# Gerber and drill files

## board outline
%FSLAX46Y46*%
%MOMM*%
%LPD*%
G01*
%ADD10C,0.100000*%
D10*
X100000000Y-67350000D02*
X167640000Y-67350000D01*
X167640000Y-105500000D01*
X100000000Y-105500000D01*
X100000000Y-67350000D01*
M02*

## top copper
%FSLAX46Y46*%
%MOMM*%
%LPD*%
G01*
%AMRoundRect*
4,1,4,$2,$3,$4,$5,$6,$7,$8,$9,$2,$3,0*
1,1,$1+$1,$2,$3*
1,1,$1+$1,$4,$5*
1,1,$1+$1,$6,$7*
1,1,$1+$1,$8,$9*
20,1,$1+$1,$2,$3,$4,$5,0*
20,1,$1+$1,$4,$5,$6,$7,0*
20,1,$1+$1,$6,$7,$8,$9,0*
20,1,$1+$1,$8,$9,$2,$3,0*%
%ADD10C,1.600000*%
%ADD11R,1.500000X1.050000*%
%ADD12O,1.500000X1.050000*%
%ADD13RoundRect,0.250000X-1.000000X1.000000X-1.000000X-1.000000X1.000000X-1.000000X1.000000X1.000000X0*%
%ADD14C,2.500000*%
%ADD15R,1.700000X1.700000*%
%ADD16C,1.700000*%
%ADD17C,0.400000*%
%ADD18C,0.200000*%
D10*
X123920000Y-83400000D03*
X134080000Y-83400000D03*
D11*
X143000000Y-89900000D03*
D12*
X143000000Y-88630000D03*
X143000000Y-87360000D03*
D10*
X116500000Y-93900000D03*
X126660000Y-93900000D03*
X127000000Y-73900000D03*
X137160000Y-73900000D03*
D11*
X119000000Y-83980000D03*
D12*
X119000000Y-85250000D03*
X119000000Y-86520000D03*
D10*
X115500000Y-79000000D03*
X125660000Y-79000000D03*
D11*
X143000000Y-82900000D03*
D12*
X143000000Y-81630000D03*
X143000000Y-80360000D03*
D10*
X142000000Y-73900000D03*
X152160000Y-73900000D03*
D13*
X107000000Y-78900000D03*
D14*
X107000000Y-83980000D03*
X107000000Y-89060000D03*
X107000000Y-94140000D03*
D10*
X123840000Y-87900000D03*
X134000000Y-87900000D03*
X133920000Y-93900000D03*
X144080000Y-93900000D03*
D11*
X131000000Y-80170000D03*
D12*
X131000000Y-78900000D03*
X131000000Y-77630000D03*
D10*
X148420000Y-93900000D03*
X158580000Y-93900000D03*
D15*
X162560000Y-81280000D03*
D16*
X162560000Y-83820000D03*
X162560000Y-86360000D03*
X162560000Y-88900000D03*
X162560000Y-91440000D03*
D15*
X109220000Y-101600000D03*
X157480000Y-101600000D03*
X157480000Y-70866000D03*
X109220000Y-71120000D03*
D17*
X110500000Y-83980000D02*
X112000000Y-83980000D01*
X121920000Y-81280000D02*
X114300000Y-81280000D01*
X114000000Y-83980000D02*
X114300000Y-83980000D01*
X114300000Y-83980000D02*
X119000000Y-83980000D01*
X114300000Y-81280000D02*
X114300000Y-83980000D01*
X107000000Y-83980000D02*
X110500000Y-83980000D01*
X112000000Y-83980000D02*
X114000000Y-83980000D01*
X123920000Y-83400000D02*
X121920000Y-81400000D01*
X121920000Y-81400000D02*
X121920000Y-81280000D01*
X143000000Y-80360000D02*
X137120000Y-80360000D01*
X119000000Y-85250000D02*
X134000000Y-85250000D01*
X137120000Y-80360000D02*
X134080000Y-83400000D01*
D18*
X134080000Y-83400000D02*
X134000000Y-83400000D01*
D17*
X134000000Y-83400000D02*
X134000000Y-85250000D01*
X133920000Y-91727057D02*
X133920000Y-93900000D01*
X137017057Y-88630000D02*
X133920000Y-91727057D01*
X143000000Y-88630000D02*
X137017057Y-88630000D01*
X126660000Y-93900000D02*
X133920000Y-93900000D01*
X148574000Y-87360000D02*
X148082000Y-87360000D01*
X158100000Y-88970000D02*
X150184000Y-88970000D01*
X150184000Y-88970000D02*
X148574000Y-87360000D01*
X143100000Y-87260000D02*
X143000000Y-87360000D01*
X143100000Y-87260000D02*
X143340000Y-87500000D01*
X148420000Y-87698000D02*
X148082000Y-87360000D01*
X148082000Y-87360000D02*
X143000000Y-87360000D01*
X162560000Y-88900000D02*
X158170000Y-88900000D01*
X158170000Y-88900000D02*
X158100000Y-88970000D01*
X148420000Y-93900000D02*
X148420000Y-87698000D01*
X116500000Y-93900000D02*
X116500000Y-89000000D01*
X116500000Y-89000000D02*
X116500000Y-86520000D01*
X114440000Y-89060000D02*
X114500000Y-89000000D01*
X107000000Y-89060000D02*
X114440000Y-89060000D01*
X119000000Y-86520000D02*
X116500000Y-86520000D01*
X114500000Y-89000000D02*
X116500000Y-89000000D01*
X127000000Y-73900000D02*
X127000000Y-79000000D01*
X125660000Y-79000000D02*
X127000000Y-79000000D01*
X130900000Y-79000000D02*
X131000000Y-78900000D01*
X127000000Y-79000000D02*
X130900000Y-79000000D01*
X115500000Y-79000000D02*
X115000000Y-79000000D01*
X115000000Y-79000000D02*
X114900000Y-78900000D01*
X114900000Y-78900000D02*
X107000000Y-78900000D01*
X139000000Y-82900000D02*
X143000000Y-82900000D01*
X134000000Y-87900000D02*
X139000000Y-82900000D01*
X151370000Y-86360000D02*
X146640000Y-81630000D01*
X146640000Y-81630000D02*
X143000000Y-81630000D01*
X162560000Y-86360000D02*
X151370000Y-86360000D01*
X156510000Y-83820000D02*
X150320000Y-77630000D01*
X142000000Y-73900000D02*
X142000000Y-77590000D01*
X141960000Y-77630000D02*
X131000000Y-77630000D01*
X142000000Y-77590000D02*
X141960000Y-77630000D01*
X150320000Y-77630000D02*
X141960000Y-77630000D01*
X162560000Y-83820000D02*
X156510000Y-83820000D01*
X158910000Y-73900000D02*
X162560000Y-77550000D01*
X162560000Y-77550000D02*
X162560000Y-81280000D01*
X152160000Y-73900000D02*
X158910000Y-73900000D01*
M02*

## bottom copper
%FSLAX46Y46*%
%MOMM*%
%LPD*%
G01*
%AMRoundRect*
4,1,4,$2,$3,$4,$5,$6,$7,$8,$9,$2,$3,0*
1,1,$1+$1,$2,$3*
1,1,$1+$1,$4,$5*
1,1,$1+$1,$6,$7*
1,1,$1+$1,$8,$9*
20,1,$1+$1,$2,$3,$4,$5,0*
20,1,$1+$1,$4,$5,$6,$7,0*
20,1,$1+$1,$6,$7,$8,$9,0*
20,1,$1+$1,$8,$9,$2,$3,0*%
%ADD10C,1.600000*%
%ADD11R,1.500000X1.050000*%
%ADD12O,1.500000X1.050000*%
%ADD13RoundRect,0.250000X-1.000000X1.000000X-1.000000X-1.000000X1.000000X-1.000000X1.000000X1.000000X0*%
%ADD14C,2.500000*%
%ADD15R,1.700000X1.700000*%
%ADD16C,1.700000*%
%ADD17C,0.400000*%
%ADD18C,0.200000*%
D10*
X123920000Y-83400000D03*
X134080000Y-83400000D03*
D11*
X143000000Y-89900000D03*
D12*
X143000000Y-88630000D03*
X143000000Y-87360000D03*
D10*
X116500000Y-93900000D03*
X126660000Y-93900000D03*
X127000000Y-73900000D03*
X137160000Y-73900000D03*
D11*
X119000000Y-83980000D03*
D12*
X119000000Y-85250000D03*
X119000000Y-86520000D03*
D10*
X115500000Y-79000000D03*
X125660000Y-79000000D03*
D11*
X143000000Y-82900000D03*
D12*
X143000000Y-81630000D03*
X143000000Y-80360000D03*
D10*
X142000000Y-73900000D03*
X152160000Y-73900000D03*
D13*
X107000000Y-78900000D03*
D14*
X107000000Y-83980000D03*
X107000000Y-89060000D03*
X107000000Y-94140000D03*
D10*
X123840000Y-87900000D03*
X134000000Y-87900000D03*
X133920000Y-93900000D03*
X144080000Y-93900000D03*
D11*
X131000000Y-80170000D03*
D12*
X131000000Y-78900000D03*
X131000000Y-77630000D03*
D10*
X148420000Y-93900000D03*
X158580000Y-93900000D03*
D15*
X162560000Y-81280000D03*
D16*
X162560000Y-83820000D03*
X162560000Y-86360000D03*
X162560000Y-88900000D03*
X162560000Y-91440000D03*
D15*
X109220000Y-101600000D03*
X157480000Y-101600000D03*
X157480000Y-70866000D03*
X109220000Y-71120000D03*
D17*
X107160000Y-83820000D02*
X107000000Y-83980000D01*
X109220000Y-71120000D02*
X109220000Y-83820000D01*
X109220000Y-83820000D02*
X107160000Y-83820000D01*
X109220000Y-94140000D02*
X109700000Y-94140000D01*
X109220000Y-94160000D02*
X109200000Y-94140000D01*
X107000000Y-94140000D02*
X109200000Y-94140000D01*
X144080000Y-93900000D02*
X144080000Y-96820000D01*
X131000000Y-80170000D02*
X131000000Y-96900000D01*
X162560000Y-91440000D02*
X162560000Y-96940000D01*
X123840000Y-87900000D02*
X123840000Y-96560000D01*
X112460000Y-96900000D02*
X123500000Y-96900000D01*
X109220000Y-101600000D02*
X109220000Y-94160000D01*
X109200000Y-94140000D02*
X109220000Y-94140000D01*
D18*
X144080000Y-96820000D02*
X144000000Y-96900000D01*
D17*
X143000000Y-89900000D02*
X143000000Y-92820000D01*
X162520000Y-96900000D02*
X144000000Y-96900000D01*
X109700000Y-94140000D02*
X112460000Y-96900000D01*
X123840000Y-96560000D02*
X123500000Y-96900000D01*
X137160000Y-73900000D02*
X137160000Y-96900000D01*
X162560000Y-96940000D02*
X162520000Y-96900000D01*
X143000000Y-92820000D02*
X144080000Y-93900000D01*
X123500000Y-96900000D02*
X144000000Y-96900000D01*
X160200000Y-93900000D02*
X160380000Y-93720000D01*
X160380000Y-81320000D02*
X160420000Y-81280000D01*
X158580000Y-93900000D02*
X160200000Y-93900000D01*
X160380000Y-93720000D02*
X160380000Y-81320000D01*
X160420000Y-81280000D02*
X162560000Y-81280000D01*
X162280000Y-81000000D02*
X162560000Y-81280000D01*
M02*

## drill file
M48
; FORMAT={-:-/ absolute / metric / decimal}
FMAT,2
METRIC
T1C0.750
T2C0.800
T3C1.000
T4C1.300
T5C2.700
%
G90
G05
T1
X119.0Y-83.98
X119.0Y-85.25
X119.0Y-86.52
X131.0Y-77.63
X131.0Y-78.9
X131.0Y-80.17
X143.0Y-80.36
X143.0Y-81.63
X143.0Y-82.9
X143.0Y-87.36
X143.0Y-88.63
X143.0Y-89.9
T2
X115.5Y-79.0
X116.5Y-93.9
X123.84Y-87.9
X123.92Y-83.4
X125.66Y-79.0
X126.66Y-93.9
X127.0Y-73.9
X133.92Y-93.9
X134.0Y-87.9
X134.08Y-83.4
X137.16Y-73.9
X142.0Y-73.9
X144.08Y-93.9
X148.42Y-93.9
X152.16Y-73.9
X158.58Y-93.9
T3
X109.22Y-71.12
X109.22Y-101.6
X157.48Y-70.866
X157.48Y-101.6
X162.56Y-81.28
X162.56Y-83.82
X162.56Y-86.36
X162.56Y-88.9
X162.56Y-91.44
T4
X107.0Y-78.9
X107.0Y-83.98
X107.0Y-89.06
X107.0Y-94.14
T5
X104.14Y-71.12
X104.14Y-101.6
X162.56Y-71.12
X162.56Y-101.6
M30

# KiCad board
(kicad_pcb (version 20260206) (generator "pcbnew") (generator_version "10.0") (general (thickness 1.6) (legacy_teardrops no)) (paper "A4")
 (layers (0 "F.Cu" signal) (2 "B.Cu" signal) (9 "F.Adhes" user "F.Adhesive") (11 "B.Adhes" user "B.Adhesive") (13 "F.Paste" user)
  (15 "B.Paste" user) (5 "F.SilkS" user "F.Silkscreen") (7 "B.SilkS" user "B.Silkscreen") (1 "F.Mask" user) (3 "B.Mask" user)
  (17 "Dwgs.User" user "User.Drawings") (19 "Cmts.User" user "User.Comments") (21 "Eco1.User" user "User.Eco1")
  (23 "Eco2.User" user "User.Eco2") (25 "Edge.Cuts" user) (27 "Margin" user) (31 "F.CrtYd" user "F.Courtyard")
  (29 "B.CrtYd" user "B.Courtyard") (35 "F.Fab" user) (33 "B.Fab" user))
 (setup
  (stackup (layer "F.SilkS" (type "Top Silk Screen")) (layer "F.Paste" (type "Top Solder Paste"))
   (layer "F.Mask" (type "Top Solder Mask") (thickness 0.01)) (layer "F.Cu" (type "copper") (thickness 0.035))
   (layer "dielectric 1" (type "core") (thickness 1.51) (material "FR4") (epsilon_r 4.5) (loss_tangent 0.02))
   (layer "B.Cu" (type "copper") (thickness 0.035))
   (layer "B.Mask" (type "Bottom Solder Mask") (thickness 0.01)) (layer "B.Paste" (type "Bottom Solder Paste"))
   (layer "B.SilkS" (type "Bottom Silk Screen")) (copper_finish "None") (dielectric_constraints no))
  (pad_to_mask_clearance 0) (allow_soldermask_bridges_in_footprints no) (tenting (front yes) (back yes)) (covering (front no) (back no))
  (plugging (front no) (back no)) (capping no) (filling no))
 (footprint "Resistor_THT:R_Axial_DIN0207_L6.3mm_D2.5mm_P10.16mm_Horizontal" (layer "F.Cu") (at 123.92 83.4)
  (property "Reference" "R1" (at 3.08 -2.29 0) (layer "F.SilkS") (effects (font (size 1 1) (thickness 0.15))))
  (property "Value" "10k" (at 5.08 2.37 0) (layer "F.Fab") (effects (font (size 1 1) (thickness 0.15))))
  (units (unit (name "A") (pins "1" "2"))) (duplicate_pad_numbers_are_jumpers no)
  (pad "1" thru_hole circle (at 0 0) (size 1.6 1.6) (drill 0.8) (layers "*.Cu" "*.Mask") (remove_unused_layers no) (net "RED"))
  (pad "2" thru_hole circle (at 10.16 0) (size 1.6 1.6) (drill 0.8) (layers "*.Cu" "*.Mask") (remove_unused_layers no) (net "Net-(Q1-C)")))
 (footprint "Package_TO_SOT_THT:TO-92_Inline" (layer "F.Cu") (at 143 89.9 90)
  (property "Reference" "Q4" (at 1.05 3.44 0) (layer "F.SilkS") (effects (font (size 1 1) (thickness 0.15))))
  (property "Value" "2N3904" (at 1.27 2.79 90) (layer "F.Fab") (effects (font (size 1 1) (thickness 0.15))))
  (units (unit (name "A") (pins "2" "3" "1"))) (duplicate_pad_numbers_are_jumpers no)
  (pad "1" thru_hole rect (at 0 0 90) (size 1.05 1.5) (drill 0.75) (layers "*.Cu" "*.Mask") (remove_unused_layers no) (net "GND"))
  (pad "2" thru_hole oval (at 1.27 0 90) (size 1.05 1.5) (drill 0.75) (layers "*.Cu" "*.Mask") (remove_unused_layers no) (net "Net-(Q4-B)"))
  (pad "3" thru_hole oval (at 2.54 0 90) (size 1.05 1.5) (drill 0.75) (layers "*.Cu" "*.Mask") (remove_unused_layers no) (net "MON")))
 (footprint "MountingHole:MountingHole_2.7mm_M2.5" (layer "F.Cu") (at 162.56 101.6)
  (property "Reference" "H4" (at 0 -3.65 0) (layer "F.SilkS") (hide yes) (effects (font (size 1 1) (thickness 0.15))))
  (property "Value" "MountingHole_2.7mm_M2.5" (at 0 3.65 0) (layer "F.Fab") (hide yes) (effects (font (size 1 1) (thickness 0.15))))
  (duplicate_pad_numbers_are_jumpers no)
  (pad "" np_thru_hole circle (at 0 0) (size 2.7 2.7) (drill 2.7) (layers "*.Cu" "*.Mask")))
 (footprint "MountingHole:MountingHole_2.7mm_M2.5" (layer "F.Cu") (at 104.14 71.12)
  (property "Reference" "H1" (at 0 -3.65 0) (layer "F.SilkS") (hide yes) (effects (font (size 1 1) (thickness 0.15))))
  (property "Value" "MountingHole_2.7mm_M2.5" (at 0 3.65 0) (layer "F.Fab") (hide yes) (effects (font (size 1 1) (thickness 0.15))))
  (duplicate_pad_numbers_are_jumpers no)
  (pad "" np_thru_hole circle (at 0 0) (size 2.7 2.7) (drill 2.7) (layers "*.Cu" "*.Mask")))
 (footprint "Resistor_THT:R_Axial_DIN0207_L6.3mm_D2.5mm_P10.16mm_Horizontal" (layer "F.Cu") (at 116.5 93.9)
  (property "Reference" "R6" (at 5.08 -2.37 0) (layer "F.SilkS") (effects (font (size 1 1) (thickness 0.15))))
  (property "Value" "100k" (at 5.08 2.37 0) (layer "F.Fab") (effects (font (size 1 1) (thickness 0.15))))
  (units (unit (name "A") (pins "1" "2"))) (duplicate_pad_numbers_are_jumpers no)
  (pad "1" thru_hole circle (at 0 0) (size 1.6 1.6) (drill 0.8) (layers "*.Cu" "*.Mask") (remove_unused_layers no) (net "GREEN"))
  (pad "2" thru_hole circle (at 10.16 0) (size 1.6 1.6) (drill 0.8) (layers "*.Cu" "*.Mask") (remove_unused_layers no) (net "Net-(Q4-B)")))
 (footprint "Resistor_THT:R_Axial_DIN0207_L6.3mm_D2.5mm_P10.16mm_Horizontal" (layer "F.Cu") (at 127 73.9)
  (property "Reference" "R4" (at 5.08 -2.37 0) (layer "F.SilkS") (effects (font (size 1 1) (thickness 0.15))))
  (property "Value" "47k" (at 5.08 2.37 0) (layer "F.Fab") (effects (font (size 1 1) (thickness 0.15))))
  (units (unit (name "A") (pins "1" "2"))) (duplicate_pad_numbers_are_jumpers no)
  (pad "1" thru_hole circle (at 0 0) (size 1.6 1.6) (drill 0.8) (layers "*.Cu" "*.Mask") (remove_unused_layers no) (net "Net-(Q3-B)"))
  (pad "2" thru_hole circle (at 10.16 0) (size 1.6 1.6) (drill 0.8) (layers "*.Cu" "*.Mask") (remove_unused_layers no) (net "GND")))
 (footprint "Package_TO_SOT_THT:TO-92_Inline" (layer "F.Cu") (at 119 83.98 -90)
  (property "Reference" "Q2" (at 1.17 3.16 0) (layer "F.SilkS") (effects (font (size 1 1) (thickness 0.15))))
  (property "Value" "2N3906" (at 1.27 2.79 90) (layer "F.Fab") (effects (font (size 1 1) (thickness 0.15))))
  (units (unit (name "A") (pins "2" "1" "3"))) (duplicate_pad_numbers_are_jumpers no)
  (pad "1" thru_hole rect (at 0 0 270) (size 1.05 1.5) (drill 0.75) (layers "*.Cu" "*.Mask") (remove_unused_layers no) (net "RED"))
  (pad "2" thru_hole oval (at 1.27 0 270) (size 1.05 1.5) (drill 0.75) (layers "*.Cu" "*.Mask") (remove_unused_layers no) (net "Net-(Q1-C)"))
  (pad "3" thru_hole oval (at 2.54 0 270) (size 1.05 1.5) (drill 0.75) (layers "*.Cu" "*.Mask") (remove_unused_layers no) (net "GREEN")))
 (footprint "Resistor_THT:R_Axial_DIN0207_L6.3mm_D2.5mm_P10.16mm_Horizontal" (layer "F.Cu") (at 115.5 79)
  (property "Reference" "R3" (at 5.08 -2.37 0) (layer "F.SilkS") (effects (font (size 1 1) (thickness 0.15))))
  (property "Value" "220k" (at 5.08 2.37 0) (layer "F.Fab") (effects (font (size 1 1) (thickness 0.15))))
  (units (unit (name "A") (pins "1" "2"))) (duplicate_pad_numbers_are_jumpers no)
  (pad "1" thru_hole circle (at 0 0) (size 1.6 1.6) (drill 0.8) (layers "*.Cu" "*.Mask") (remove_unused_layers no) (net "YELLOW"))
  (pad "2" thru_hole circle (at 10.16 0) (size 1.6 1.6) (drill 0.8) (layers "*.Cu" "*.Mask") (remove_unused_layers no) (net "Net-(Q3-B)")))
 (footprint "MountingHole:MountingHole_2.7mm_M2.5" (layer "F.Cu") (at 162.56 71.12)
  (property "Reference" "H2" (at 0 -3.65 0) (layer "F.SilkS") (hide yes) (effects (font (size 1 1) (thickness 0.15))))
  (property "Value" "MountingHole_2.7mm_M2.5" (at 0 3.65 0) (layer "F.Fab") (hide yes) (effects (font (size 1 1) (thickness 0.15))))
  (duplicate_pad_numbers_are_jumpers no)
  (pad "" np_thru_hole circle (at 0 0) (size 2.7 2.7) (drill 2.7) (layers "*.Cu" "*.Mask")))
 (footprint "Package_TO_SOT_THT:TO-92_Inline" (layer "F.Cu") (at 143 82.9 90)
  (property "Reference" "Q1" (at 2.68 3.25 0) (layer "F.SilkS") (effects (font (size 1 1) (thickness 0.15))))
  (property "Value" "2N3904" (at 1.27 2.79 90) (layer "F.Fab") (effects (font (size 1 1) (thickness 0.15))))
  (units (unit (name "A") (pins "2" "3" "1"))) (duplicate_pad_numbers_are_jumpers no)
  (pad "1" thru_hole rect (at 0 0 90) (size 1.05 1.5) (drill 0.75) (layers "*.Cu" "*.Mask") (remove_unused_layers no) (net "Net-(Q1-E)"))
  (pad "2" thru_hole oval (at 1.27 0 90) (size 1.05 1.5) (drill 0.75) (layers "*.Cu" "*.Mask") (remove_unused_layers no) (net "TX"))
  (pad "3" thru_hole oval (at 2.54 0 90) (size 1.05 1.5) (drill 0.75) (layers "*.Cu" "*.Mask") (remove_unused_layers no) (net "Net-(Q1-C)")))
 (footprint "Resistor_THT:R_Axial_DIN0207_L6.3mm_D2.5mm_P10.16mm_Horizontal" (layer "F.Cu") (at 142 73.9)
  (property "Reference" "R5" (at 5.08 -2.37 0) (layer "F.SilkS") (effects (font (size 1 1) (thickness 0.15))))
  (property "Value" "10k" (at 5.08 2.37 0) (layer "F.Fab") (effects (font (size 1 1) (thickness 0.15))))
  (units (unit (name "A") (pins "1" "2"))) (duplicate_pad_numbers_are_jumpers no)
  (pad "1" thru_hole circle (at 0 0) (size 1.6 1.6) (drill 0.8) (layers "*.Cu" "*.Mask") (remove_unused_layers no) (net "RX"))
  (pad "2" thru_hole circle (at 10.16 0) (size 1.6 1.6) (drill 0.8) (layers "*.Cu" "*.Mask") (remove_unused_layers no) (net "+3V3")))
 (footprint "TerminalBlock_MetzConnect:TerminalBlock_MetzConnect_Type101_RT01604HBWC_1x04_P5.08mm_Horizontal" (layer "F.Cu")
  (at 107 78.9 -90)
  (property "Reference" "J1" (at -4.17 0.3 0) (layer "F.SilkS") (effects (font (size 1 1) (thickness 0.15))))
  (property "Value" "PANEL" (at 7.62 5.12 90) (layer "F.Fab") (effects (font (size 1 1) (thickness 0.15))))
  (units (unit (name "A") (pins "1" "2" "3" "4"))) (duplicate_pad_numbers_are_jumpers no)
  (pad "1" thru_hole roundrect (at 0 0 270) (size 2.5 2.5) (drill 1.3) (layers "*.Cu" "*.Mask") (remove_unused_layers no)
   (roundrect_rratio 0.1) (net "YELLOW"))
  (pad "2" thru_hole circle (at 5.08 0 270) (size 2.5 2.5) (drill 1.3) (layers "*.Cu" "*.Mask") (remove_unused_layers no) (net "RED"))
  (pad "3" thru_hole circle (at 10.16 0 270) (size 2.5 2.5) (drill 1.3) (layers "*.Cu" "*.Mask") (remove_unused_layers no) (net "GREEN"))
  (pad "4" thru_hole circle (at 15.24 0 270) (size 2.5 2.5) (drill 1.3) (layers "*.Cu" "*.Mask") (remove_unused_layers no) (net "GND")))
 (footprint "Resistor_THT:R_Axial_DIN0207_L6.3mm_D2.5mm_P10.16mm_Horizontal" (layer "F.Cu") (at 123.84 87.9)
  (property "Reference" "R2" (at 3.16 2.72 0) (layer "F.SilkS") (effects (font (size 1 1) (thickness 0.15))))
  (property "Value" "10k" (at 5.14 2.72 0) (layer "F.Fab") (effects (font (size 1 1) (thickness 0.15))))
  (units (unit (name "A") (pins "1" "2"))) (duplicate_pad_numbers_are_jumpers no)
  (pad "1" thru_hole circle (at 0 0) (size 1.6 1.6) (drill 0.8) (layers "*.Cu" "*.Mask") (remove_unused_layers no) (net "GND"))
  (pad "2" thru_hole circle (at 10.16 0) (size 1.6 1.6) (drill 0.8) (layers "*.Cu" "*.Mask") (remove_unused_layers no) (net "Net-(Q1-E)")))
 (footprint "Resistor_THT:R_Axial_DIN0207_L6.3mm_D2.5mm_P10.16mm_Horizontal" (layer "F.Cu") (at 133.92 93.9)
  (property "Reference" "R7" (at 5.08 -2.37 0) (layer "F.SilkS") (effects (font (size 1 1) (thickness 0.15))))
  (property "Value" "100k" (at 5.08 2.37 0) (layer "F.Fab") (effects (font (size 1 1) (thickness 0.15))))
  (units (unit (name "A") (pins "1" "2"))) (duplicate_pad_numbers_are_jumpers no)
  (pad "1" thru_hole circle (at 0 0) (size 1.6 1.6) (drill 0.8) (layers "*.Cu" "*.Mask") (remove_unused_layers no) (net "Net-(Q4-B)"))
  (pad "2" thru_hole circle (at 10.16 0) (size 1.6 1.6) (drill 0.8) (layers "*.Cu" "*.Mask") (remove_unused_layers no) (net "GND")))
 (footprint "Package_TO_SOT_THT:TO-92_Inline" (layer "F.Cu") (at 131 80.17 90)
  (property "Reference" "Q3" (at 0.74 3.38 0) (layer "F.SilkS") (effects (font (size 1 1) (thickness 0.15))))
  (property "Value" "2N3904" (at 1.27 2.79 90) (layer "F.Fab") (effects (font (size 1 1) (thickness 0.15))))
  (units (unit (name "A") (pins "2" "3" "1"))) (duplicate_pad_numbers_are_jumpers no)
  (pad "1" thru_hole rect (at 0 0 90) (size 1.05 1.5) (drill 0.75) (layers "*.Cu" "*.Mask") (remove_unused_layers no) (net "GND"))
  (pad "2" thru_hole oval (at 1.27 0 90) (size 1.05 1.5) (drill 0.75) (layers "*.Cu" "*.Mask") (remove_unused_layers no) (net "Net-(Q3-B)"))
  (pad "3" thru_hole oval (at 2.54 0 90) (size 1.05 1.5) (drill 0.75) (layers "*.Cu" "*.Mask") (remove_unused_layers no) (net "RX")))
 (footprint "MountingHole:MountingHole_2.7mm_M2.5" (layer "F.Cu") (at 104.14 101.6)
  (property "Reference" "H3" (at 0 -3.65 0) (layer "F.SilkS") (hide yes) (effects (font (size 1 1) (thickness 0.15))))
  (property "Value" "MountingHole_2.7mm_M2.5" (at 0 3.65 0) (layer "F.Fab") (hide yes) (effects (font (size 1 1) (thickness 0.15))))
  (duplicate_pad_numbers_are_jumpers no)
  (pad "" np_thru_hole circle (at 0 0) (size 2.7 2.7) (drill 2.7) (layers "*.Cu" "*.Mask")))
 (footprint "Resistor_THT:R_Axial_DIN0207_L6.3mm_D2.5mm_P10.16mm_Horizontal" (layer "F.Cu") (at 148.42 93.9)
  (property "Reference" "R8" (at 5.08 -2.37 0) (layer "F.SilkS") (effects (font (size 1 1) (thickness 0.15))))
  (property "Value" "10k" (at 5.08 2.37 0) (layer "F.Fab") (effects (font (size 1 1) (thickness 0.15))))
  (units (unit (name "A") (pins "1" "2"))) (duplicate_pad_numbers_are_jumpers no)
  (pad "1" thru_hole circle (at 0 0) (size 1.6 1.6) (drill 0.8) (layers "*.Cu" "*.Mask") (remove_unused_layers no) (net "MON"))
  (pad "2" thru_hole circle (at 10.16 0) (size 1.6 1.6) (drill 0.8) (layers "*.Cu" "*.Mask") (remove_unused_layers no) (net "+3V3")))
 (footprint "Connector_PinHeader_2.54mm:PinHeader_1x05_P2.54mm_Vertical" (layer "F.Cu") (at 162.56 81.28)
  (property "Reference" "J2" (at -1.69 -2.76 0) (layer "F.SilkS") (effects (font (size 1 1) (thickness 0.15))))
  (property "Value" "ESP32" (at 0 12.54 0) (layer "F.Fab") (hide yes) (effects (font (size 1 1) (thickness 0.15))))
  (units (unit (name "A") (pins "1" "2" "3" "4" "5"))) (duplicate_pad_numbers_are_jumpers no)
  (pad "1" thru_hole rect (at 0 0) (size 1.7 1.7) (drill 1) (layers "*.Cu" "*.Mask") (remove_unused_layers no) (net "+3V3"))
  (pad "2" thru_hole circle (at 0 2.54) (size 1.7 1.7) (drill 1) (layers "*.Cu" "*.Mask") (remove_unused_layers no) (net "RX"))
  (pad "3" thru_hole circle (at 0 5.08) (size 1.7 1.7) (drill 1) (layers "*.Cu" "*.Mask") (remove_unused_layers no) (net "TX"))
  (pad "4" thru_hole circle (at 0 7.62) (size 1.7 1.7) (drill 1) (layers "*.Cu" "*.Mask") (remove_unused_layers no) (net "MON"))
  (pad "5" thru_hole circle (at 0 10.16) (size 1.7 1.7) (drill 1) (layers "*.Cu" "*.Mask") (remove_unused_layers no) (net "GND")))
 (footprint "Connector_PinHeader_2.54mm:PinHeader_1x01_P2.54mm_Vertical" (layer "B.Cu") (at 109.22 101.6)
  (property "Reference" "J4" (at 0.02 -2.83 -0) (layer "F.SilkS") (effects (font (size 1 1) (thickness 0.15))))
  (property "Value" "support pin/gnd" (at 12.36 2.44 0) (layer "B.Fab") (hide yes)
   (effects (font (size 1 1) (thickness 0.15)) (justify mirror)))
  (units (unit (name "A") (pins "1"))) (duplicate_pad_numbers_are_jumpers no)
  (pad "1" thru_hole rect (at 0 0) (size 1.7 1.7) (drill 1) (layers "*.Cu" "*.Mask") (remove_unused_layers no) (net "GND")))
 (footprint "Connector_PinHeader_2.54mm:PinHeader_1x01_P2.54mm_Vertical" (layer "B.Cu") (at 157.48 101.6)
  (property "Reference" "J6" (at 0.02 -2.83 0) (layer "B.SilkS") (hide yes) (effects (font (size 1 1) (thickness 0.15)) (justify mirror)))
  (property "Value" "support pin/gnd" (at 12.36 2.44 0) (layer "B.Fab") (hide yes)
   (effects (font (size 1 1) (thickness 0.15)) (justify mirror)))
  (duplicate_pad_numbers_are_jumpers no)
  (pad "1" thru_hole rect (at 0 0) (size 1.7 1.7) (drill 1) (layers "*.Cu" "*.Mask") (remove_unused_layers no)))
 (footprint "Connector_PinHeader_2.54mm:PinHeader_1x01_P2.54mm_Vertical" (layer "B.Cu") (at 157.48 70.866)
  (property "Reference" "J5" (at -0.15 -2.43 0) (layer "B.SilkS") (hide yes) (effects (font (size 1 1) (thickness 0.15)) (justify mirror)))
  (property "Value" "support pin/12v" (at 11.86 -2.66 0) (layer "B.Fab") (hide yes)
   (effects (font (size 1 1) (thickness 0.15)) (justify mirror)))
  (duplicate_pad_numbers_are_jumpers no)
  (pad "1" thru_hole rect (at 0 0) (size 1.7 1.7) (drill 1) (layers "*.Cu" "*.Mask") (remove_unused_layers no)))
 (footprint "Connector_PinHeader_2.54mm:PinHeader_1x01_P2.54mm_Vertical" (layer "B.Cu") (at 109.22 71.12)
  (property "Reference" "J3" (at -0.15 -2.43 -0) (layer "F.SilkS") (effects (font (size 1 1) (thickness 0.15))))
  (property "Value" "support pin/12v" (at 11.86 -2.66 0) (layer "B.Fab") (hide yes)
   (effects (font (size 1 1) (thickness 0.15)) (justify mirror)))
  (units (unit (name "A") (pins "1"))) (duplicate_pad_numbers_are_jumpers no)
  (pad "1" thru_hole rect (at 0 0) (size 1.7 1.7) (drill 1) (layers "*.Cu" "*.Mask") (remove_unused_layers no) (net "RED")))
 (gr_rect (start 100 67.35) (end 167.64 105.5) (stroke (width 0.1) (type default)) (fill no) (layer "Edge.Cuts"))
 (segment (start 110.5 83.98) (end 112 83.98) (width 0.4) (layer "F.Cu") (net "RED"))
 (segment (start 121.92 81.28) (end 114.3 81.28) (width 0.4) (layer "F.Cu") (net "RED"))
 (segment (start 114 83.98) (end 114.3 83.98) (width 0.4) (layer "F.Cu") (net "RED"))
 (segment (start 114.3 83.98) (end 119 83.98) (width 0.4) (layer "F.Cu") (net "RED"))
 (segment (start 114.3 81.28) (end 114.3 83.98) (width 0.4) (layer "F.Cu") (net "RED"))
 (segment (start 107 83.98) (end 110.5 83.98) (width 0.4) (layer "F.Cu") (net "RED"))
 (segment (start 112 83.98) (end 114 83.98) (width 0.4) (layer "F.Cu") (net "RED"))
 (segment (start 123.92 83.4) (end 121.92 81.4) (width 0.4) (layer "F.Cu") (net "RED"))
 (segment (start 121.92 81.4) (end 121.92 81.28) (width 0.4) (layer "F.Cu") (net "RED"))
 (segment (start 107.16 83.82) (end 107 83.98) (width 0.4) (layer "B.Cu") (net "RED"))
 (segment (start 109.22 71.12) (end 109.22 83.82) (width 0.4) (layer "B.Cu") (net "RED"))
 (segment (start 109.22 83.82) (end 107.16 83.82) (width 0.4) (layer "B.Cu") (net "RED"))
 (segment (start 143 80.36) (end 137.12 80.36) (width 0.4) (layer "F.Cu") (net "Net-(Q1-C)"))
 (segment (start 119 85.25) (end 134 85.25) (width 0.4) (layer "F.Cu") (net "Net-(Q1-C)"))
 (segment (start 137.12 80.36) (end 134.08 83.4) (width 0.4) (layer "F.Cu") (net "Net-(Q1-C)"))
 (segment (start 134.08 83.4) (end 134 83.4) (width 0.2) (layer "F.Cu") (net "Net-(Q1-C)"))
 (segment (start 134 83.4) (end 134 85.25) (width 0.4) (layer "F.Cu") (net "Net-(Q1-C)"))
 (segment (start 109.22 94.14) (end 109.7 94.14) (width 0.4) (layer "B.Cu") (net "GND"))
 (segment (start 109.22 94.16) (end 109.2 94.14) (width 0.4) (layer "B.Cu") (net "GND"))
 (segment (start 107 94.14) (end 109.2 94.14) (width 0.4) (layer "B.Cu") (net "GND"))
 (segment (start 144.08 93.9) (end 144.08 96.82) (width 0.4) (layer "B.Cu") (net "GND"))
 (segment (start 131 80.17) (end 131 96.9) (width 0.4) (layer "B.Cu") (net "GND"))
 (segment (start 162.56 91.44) (end 162.56 96.94) (width 0.4) (layer "B.Cu") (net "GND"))
 (segment (start 123.84 87.9) (end 123.84 96.56) (width 0.4) (layer "B.Cu") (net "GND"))
 (segment (start 112.46 96.9) (end 123.5 96.9) (width 0.4) (layer "B.Cu") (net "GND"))
 (segment (start 109.22 101.6) (end 109.22 94.16) (width 0.4) (layer "B.Cu") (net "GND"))
 (segment (start 109.2 94.14) (end 109.22 94.14) (width 0.4) (layer "B.Cu") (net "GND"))
 (segment (start 144.08 96.82) (end 144 96.9) (width 0.2) (layer "B.Cu") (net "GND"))
 (segment (start 143 89.9) (end 143 92.82) (width 0.4) (layer "B.Cu") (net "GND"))
 (segment (start 162.52 96.9) (end 144 96.9) (width 0.4) (layer "B.Cu") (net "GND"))
 (segment (start 109.7 94.14) (end 112.46 96.9) (width 0.4) (layer "B.Cu") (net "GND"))
 (segment (start 123.84 96.56) (end 123.5 96.9) (width 0.4) (layer "B.Cu") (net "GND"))
 (segment (start 137.16 73.9) (end 137.16 96.9) (width 0.4) (layer "B.Cu") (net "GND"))
 (segment (start 162.56 96.94) (end 162.52 96.9) (width 0.4) (layer "B.Cu") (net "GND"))
 (segment (start 143 92.82) (end 144.08 93.9) (width 0.4) (layer "B.Cu") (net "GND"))
 (segment (start 123.5 96.9) (end 144 96.9) (width 0.4) (layer "B.Cu") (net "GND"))
 (segment (start 133.92 91.727057) (end 133.92 93.9) (width 0.4) (layer "F.Cu") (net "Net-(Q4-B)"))
 (segment (start 137.017057 88.63) (end 133.92 91.727057) (width 0.4) (layer "F.Cu") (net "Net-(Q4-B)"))
 (segment (start 143 88.63) (end 137.017057 88.63) (width 0.4) (layer "F.Cu") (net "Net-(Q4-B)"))
 (segment (start 126.66 93.9) (end 133.92 93.9) (width 0.4) (layer "F.Cu") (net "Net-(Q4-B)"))
 (segment (start 148.574 87.36) (end 148.082 87.36) (width 0.4) (layer "F.Cu") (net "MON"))
 (segment (start 158.1 88.97) (end 150.184 88.97) (width 0.4) (layer "F.Cu") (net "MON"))
 (segment (start 150.184 88.97) (end 148.574 87.36) (width 0.4) (layer "F.Cu") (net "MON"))
 (segment (start 143.1 87.26) (end 143 87.36) (width 0.4) (layer "F.Cu") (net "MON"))
 (segment (start 143.1 87.26) (end 143.34 87.5) (width 0.4) (layer "F.Cu") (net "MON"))
 (segment (start 148.42 87.698) (end 148.082 87.36) (width 0.4) (layer "F.Cu") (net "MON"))
 (segment (start 148.082 87.36) (end 143 87.36) (width 0.4) (layer "F.Cu") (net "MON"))
 (segment (start 162.56 88.9) (end 158.17 88.9) (width 0.4) (layer "F.Cu") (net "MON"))
 (segment (start 158.17 88.9) (end 158.1 88.97) (width 0.4) (layer "F.Cu") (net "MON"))
 (segment (start 148.42 93.9) (end 148.42 87.698) (width 0.4) (layer "F.Cu") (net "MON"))
 (segment (start 116.5 93.9) (end 116.5 89) (width 0.4) (layer "F.Cu") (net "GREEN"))
 (segment (start 116.5 89) (end 116.5 86.52) (width 0.4) (layer "F.Cu") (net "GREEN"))
 (segment (start 114.44 89.06) (end 114.5 89) (width 0.4) (layer "F.Cu") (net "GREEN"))
 (segment (start 107 89.06) (end 114.44 89.06) (width 0.4) (layer "F.Cu") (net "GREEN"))
 (segment (start 119 86.52) (end 116.5 86.52) (width 0.4) (layer "F.Cu") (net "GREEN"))
 (segment (start 114.5 89) (end 116.5 89) (width 0.4) (layer "F.Cu") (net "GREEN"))
 (segment (start 127 73.9) (end 127 79) (width 0.4) (layer "F.Cu") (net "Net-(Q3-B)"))
 (segment (start 125.66 79) (end 127 79) (width 0.4) (layer "F.Cu") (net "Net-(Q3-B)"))
 (segment (start 130.9 79) (end 131 78.9) (width 0.4) (layer "F.Cu") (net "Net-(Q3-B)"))
 (segment (start 127 79) (end 130.9 79) (width 0.4) (layer "F.Cu") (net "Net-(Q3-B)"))
 (segment (start 115.5 79) (end 115 79) (width 0.4) (layer "F.Cu") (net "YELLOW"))
 (segment (start 115 79) (end 114.9 78.9) (width 0.4) (layer "F.Cu") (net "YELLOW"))
 (segment (start 114.9 78.9) (end 107 78.9) (width 0.4) (layer "F.Cu") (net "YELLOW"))
 (segment (start 139 82.9) (end 143 82.9) (width 0.4) (layer "F.Cu") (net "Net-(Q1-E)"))
 (segment (start 134 87.9) (end 139 82.9) (width 0.4) (layer "F.Cu") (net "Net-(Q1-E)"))
 (segment (start 151.37 86.36) (end 146.64 81.63) (width 0.4) (layer "F.Cu") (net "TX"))
 (segment (start 146.64 81.63) (end 143 81.63) (width 0.4) (layer "F.Cu") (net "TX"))
 (segment (start 162.56 86.36) (end 151.37 86.36) (width 0.4) (layer "F.Cu") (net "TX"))
 (segment (start 156.51 83.82) (end 150.32 77.63) (width 0.4) (layer "F.Cu") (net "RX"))
 (segment (start 142 73.9) (end 142 77.59) (width 0.4) (layer "F.Cu") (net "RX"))
 (segment (start 141.96 77.63) (end 131 77.63) (width 0.4) (layer "F.Cu") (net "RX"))
 (segment (start 142 77.59) (end 141.96 77.63) (width 0.4) (layer "F.Cu") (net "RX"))
 (segment (start 150.32 77.63) (end 141.96 77.63) (width 0.4) (layer "F.Cu") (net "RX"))
 (segment (start 162.56 83.82) (end 156.51 83.82) (width 0.4) (layer "F.Cu") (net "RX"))
 (segment (start 158.91 73.9) (end 162.56 77.55) (width 0.4) (layer "F.Cu") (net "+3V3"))
 (segment (start 162.56 77.55) (end 162.56 81.28) (width 0.4) (layer "F.Cu") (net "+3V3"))
 (segment (start 152.16 73.9) (end 158.91 73.9) (width 0.4) (layer "F.Cu") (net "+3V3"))
 (segment (start 160.2 93.9) (end 160.38 93.72) (width 0.4) (layer "B.Cu") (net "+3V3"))
 (segment (start 160.38 81.32) (end 160.42 81.28) (width 0.4) (layer "B.Cu") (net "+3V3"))
 (segment (start 158.58 93.9) (end 160.2 93.9) (width 0.4) (layer "B.Cu") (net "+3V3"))
 (segment (start 160.38 93.72) (end 160.38 81.32) (width 0.4) (layer "B.Cu") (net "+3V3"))
 (segment (start 160.42 81.28) (end 162.56 81.28) (width 0.4) (layer "B.Cu") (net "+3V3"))
 (segment (start 162.28 81) (end 162.56 81.28) (width 0.4) (layer "B.Cu") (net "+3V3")))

